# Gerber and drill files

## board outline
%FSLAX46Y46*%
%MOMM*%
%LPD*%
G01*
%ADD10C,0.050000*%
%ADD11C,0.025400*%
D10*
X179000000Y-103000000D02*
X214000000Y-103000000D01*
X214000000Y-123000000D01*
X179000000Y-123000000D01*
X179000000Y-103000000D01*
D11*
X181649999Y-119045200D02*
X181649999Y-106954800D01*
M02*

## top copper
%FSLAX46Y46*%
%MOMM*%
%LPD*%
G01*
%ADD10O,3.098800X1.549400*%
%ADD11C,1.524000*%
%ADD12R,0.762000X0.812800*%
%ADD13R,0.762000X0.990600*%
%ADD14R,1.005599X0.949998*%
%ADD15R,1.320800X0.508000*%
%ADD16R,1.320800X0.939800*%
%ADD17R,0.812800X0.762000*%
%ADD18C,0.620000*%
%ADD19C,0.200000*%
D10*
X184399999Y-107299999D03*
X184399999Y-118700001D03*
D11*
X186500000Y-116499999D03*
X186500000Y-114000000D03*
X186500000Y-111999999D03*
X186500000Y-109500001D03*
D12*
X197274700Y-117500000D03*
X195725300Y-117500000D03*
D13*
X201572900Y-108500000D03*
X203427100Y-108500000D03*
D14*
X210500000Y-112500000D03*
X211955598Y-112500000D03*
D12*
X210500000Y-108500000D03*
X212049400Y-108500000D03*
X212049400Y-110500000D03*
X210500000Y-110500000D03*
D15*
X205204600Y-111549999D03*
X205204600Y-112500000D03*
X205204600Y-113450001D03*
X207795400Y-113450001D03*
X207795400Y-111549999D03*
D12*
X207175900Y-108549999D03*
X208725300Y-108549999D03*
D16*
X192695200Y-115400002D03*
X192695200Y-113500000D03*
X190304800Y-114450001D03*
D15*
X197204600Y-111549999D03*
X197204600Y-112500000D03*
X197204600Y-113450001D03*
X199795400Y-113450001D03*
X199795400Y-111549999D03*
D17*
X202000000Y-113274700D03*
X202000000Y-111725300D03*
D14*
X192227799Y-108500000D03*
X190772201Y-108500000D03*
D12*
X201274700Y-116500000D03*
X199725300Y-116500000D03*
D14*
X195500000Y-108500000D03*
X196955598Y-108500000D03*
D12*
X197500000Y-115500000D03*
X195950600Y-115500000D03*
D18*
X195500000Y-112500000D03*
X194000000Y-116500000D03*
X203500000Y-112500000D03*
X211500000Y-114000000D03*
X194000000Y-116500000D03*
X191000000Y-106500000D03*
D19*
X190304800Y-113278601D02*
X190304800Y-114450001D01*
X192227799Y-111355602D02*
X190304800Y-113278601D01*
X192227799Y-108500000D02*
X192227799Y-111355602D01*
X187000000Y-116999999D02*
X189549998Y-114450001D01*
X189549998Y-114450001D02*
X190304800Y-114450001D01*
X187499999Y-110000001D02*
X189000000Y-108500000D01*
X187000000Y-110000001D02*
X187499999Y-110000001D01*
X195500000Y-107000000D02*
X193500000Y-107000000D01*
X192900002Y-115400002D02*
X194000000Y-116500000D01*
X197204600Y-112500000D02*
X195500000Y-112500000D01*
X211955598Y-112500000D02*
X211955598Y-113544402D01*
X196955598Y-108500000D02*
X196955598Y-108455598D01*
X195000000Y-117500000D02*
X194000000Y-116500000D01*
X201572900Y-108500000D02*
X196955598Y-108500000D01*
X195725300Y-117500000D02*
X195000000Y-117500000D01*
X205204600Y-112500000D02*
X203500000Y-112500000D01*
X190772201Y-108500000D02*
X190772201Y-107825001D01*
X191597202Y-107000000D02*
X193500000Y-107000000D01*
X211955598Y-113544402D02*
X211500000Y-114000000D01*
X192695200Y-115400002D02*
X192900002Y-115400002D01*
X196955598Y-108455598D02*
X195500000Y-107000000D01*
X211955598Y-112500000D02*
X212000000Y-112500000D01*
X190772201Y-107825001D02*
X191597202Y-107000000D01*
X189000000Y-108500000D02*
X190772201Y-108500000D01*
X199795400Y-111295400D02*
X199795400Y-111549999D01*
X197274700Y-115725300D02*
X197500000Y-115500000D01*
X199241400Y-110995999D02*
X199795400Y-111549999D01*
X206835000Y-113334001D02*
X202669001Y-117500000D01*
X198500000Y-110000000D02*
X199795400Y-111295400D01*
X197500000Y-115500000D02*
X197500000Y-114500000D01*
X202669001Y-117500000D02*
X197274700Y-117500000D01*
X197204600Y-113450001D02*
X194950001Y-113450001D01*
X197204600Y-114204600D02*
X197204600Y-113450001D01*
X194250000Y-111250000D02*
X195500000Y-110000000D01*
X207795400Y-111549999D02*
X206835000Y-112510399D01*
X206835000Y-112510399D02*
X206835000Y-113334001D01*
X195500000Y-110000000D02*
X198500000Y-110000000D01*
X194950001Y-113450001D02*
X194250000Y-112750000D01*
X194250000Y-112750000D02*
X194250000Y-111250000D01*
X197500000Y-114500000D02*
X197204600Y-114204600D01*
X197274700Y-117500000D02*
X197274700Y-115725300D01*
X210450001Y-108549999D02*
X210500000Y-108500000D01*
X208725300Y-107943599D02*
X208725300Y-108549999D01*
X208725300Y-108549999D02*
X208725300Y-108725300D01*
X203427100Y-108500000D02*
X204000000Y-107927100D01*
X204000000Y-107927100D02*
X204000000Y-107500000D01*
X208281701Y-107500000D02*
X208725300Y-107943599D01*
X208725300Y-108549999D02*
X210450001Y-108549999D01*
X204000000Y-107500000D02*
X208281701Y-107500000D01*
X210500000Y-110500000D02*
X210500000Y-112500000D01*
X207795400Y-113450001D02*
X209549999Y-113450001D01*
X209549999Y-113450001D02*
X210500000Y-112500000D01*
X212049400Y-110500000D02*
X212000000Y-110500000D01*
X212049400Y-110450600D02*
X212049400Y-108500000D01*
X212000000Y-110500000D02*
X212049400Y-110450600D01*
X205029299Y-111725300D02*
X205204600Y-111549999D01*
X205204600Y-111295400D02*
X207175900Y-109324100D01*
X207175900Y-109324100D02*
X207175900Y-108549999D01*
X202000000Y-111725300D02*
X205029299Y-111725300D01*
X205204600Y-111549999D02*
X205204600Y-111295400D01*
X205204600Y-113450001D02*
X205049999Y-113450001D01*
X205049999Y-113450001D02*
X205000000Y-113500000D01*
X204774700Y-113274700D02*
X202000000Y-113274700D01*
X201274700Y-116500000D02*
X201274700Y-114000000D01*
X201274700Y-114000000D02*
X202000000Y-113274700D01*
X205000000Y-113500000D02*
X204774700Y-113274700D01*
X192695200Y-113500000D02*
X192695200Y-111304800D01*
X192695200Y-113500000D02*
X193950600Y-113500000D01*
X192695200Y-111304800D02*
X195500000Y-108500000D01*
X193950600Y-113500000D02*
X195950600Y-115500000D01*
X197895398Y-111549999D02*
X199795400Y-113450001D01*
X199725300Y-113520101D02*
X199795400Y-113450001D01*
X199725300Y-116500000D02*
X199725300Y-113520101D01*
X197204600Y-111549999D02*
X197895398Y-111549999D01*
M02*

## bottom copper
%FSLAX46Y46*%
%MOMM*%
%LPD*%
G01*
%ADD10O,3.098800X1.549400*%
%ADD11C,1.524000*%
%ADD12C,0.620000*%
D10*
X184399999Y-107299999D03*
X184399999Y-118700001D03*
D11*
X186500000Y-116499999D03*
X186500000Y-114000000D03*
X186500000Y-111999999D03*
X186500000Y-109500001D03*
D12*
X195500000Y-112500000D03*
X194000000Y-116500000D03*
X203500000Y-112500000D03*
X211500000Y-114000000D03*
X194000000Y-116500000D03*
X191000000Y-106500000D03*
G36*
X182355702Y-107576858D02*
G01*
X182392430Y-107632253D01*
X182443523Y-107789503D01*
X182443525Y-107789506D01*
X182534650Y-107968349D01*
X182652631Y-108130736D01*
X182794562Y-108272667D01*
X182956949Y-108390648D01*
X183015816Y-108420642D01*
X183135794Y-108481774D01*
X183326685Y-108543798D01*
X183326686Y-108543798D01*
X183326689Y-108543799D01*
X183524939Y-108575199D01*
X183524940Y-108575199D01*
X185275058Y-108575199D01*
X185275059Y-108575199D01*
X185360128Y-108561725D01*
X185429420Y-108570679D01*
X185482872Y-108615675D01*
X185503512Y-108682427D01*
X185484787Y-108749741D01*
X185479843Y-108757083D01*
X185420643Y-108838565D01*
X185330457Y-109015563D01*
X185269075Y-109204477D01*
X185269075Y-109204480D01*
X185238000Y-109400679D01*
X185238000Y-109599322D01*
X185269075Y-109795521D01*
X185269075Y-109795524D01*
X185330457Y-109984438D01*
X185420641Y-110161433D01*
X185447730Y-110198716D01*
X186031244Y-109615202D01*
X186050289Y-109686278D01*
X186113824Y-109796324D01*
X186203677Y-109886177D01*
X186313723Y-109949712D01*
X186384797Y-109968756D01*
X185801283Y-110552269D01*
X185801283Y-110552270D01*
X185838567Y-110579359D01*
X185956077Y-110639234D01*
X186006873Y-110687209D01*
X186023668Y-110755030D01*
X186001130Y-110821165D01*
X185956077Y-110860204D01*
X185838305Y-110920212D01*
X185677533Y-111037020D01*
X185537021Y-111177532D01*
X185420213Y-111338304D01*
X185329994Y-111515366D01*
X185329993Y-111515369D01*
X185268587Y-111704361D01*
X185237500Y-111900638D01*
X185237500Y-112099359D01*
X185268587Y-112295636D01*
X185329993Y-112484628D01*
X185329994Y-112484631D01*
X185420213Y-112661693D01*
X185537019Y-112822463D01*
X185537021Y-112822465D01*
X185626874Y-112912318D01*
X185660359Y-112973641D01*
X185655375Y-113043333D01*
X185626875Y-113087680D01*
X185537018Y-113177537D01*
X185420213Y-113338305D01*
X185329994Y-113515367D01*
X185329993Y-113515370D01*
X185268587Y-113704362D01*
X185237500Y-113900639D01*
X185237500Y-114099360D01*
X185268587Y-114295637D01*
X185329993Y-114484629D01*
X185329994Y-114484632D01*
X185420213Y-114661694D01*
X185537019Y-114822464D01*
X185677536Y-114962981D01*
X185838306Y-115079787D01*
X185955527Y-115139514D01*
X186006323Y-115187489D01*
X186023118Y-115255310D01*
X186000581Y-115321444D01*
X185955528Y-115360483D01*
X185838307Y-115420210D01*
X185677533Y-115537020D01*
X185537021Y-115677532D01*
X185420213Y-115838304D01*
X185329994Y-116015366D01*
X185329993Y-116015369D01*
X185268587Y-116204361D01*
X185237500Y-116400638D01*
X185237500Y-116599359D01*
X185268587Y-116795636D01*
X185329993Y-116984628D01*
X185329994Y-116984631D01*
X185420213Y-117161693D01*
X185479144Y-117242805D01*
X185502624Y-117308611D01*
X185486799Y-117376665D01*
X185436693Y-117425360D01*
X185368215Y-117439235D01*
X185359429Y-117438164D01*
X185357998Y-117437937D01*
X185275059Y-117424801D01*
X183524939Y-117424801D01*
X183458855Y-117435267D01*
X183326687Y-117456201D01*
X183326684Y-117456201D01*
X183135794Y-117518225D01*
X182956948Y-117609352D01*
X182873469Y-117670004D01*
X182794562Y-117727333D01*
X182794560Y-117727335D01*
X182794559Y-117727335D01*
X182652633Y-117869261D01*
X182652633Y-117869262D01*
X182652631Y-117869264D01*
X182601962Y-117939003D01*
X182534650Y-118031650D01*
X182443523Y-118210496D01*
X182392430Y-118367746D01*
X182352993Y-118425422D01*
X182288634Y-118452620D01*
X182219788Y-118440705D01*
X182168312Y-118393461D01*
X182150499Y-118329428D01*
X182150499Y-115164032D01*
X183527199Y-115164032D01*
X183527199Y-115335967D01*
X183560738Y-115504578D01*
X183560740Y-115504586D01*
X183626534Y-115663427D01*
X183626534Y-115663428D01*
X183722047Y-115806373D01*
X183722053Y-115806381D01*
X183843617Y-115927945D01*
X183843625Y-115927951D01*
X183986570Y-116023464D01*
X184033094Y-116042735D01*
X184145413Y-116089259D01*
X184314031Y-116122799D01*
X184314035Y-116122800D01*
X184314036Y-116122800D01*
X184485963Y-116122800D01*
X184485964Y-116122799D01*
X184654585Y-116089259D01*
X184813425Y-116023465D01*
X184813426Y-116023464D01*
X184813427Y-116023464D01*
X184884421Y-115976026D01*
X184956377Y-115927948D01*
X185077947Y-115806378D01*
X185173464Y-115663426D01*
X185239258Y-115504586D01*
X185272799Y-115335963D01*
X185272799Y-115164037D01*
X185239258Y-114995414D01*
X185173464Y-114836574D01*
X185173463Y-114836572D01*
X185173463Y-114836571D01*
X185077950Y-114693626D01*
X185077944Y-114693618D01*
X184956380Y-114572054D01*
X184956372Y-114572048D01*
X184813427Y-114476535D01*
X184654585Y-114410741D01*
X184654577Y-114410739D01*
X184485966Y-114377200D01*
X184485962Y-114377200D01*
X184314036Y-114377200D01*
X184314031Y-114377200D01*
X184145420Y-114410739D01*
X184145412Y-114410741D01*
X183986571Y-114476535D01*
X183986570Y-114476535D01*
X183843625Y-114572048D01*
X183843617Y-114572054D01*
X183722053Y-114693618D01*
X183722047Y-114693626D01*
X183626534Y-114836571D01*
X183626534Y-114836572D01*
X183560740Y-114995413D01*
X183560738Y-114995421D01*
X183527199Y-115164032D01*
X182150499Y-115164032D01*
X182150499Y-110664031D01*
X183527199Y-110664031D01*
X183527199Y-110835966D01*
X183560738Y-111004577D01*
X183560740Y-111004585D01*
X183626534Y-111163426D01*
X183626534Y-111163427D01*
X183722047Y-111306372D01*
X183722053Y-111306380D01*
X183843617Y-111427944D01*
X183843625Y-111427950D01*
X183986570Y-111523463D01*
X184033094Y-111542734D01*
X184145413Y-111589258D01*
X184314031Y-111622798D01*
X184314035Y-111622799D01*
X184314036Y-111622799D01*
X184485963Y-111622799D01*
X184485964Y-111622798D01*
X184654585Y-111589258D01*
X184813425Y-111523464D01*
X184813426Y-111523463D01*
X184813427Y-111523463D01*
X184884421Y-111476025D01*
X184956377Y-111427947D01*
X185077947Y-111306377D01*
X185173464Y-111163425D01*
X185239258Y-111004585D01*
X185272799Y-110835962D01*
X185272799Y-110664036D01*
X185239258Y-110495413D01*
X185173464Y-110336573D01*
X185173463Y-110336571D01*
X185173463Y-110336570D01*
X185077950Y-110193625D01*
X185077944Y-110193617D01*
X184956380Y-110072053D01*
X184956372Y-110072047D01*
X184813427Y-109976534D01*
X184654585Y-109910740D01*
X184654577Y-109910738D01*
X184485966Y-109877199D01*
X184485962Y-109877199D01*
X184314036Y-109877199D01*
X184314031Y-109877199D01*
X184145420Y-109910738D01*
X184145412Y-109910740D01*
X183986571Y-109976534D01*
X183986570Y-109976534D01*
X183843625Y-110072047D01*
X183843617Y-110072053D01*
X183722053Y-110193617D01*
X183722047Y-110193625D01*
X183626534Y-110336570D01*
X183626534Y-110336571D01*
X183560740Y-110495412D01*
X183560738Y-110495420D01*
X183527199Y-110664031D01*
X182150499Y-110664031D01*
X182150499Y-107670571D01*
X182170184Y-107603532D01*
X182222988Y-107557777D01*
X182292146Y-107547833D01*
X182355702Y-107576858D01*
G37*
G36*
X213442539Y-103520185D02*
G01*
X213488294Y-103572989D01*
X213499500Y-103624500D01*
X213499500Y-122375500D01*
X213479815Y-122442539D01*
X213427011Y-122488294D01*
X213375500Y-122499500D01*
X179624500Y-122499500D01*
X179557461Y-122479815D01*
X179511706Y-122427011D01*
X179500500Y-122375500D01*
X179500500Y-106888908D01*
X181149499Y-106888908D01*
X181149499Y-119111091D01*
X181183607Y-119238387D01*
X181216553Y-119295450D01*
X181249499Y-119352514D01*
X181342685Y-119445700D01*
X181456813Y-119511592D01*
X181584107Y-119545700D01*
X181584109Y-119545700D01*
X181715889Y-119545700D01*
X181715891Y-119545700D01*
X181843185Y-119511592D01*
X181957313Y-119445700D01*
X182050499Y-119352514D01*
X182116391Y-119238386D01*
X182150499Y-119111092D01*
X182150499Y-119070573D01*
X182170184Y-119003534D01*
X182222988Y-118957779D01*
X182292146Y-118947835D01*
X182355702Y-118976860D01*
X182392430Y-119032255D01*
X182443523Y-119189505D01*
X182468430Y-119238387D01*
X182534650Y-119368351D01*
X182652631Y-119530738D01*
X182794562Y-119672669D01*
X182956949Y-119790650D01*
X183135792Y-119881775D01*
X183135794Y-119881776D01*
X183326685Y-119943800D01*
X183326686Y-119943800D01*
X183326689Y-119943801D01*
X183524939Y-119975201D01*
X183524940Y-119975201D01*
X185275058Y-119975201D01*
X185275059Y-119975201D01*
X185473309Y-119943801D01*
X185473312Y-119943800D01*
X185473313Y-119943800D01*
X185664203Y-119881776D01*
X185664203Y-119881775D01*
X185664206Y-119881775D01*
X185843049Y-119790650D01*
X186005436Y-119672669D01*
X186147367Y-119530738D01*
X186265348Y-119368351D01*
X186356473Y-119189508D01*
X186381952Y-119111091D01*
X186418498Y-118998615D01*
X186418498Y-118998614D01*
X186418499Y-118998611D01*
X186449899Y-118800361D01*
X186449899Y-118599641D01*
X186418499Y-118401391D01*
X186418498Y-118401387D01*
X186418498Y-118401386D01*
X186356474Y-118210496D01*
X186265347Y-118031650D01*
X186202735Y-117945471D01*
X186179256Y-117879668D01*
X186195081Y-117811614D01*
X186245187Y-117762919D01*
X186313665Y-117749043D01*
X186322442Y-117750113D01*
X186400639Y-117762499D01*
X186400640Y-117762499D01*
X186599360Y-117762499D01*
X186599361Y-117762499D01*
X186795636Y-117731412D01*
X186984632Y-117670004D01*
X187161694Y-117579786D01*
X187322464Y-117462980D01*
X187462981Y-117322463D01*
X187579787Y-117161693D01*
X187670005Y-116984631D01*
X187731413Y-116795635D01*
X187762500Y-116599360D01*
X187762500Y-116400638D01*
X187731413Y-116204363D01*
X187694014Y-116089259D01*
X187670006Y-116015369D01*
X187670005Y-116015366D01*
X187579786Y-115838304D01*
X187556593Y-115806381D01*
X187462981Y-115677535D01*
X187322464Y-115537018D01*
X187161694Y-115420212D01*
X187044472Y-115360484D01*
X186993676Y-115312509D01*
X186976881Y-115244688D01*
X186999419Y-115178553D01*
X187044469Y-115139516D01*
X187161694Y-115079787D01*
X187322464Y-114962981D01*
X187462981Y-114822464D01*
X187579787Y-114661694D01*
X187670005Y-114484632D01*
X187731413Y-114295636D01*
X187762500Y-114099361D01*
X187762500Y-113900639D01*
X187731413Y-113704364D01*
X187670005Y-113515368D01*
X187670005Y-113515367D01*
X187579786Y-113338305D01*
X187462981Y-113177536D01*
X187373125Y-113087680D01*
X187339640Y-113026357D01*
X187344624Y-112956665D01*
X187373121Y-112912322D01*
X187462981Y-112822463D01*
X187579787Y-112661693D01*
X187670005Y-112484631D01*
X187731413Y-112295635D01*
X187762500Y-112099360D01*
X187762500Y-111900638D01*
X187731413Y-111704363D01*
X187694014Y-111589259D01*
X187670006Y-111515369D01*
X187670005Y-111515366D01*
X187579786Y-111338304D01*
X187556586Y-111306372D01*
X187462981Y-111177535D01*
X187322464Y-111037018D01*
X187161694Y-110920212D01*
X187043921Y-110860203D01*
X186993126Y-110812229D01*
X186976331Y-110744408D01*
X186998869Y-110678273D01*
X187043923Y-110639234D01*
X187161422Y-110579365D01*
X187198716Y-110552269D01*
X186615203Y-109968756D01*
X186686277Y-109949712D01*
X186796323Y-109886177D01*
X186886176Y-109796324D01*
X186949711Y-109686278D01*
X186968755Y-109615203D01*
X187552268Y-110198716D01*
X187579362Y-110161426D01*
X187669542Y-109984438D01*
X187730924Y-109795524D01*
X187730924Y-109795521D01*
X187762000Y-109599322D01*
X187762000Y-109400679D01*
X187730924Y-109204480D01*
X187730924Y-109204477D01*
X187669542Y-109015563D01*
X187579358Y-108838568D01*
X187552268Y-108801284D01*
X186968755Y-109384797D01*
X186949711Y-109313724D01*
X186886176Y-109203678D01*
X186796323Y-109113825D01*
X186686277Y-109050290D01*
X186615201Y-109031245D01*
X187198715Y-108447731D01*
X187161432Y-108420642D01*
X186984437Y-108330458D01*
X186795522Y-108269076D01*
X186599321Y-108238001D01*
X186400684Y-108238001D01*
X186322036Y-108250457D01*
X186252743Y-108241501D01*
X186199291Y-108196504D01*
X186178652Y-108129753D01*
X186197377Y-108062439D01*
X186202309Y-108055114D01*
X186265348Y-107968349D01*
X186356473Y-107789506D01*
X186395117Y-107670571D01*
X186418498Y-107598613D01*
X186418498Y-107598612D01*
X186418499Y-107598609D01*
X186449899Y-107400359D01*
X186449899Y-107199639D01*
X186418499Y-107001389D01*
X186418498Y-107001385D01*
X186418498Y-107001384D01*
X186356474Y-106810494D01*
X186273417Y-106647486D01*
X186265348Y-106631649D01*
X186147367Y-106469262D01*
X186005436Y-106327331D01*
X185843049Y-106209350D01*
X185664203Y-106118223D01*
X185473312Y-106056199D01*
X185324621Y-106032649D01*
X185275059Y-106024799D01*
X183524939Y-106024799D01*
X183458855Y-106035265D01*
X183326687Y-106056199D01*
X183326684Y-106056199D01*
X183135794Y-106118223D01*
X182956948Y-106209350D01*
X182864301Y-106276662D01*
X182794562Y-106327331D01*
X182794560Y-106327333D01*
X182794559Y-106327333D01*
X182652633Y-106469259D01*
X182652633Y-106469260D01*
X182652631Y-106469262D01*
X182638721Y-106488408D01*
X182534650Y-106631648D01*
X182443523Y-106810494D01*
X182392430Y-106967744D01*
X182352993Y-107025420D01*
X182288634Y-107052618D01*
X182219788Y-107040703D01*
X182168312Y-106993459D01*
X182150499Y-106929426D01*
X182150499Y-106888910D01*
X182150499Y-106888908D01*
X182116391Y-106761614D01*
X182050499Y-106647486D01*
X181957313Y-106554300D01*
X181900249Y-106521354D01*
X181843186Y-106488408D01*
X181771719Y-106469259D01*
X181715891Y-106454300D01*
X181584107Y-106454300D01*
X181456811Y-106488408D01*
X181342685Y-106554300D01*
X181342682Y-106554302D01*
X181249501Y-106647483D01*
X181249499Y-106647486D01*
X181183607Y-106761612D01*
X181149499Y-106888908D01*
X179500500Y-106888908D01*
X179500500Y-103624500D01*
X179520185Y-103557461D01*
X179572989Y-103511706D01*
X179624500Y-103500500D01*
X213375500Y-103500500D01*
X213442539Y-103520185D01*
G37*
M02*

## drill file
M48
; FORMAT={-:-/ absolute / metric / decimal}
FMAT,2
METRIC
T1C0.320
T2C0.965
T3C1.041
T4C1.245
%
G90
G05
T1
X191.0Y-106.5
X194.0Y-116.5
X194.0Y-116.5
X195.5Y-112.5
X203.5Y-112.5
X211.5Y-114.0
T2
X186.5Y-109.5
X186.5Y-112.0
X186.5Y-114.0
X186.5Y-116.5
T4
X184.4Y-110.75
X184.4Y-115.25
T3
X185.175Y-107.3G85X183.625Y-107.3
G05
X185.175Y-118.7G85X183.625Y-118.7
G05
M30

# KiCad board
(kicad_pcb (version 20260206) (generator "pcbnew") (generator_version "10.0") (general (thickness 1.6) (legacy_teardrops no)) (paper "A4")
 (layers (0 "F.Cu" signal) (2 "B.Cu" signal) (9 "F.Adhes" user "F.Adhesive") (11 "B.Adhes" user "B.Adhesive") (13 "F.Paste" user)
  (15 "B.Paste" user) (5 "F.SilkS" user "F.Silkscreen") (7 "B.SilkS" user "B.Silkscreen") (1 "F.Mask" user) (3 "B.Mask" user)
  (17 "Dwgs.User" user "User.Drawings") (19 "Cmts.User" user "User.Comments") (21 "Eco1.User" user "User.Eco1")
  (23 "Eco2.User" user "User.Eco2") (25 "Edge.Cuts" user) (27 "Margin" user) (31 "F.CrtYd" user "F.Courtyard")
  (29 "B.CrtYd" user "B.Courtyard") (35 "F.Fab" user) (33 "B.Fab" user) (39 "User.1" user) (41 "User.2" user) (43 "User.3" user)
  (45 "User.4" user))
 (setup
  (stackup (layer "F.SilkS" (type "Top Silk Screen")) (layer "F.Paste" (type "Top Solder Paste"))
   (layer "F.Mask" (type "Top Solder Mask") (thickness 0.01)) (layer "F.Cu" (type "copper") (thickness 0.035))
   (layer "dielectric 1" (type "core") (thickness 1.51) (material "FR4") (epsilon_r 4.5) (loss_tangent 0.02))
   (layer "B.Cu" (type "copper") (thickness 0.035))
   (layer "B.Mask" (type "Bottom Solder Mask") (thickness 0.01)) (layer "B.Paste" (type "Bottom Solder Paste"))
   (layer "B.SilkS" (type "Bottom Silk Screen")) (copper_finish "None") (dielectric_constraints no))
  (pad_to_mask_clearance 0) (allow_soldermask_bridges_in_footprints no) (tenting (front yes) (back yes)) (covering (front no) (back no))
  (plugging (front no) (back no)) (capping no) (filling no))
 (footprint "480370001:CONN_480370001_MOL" (layer "F.Cu") (at 186.5 116.499999 -90)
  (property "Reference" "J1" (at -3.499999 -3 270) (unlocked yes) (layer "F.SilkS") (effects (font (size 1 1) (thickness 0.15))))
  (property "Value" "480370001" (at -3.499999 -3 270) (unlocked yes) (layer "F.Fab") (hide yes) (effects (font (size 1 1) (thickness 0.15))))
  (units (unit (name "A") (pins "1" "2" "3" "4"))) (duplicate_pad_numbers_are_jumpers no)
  (fp_line (start 2.545201 4.850001) (end -9.545199 4.850001) (stroke (width 0.0254) (type solid)) (layer "Edge.Cuts"))
  (pad "" np_thru_hole oval (at -9.2 2.100001 270) (size 1.5494 3.0988) (drill oval 1.0414 2.5908) (layers "*.Cu" "*.Mask"))
  (pad "" np_thru_hole circle (at -5.75 2.100001 270) (size 1.2446 1.2446) (drill 1.2446) (layers))
  (pad "" np_thru_hole circle (at -1.249999 2.100001 270) (size 1.2446 1.2446) (drill 1.2446) (layers))
  (pad "" np_thru_hole oval (at 2.200002 2.100001 270) (size 1.5494 3.0988) (drill oval 1.0414 2.5908) (layers "*.Cu" "*.Mask"))
  (pad "1" thru_hole circle (at 0 0 270) (size 1.524 1.524) (drill 0.9652) (layers "*.Cu" "*.Mask") (remove_unused_layers no)
   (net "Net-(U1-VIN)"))
  (pad "2" thru_hole circle (at -2.499999 0 270) (size 1.524 1.524) (drill 0.9652) (layers "*.Cu" "*.Mask") (remove_unused_layers no)
   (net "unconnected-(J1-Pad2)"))
  (pad "3" thru_hole circle (at -4.5 0 270) (size 1.524 1.524) (drill 0.9652) (layers "*.Cu" "*.Mask") (remove_unused_layers no)
   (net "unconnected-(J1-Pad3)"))
  (pad "4" thru_hole circle (at -6.999998 0 270) (size 1.524 1.524) (drill 0.9652) (layers "*.Cu" "*.Mask") (remove_unused_layers no)
   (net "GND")))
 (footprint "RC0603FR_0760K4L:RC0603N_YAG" (layer "F.Cu") (at 196.5 117.5 180)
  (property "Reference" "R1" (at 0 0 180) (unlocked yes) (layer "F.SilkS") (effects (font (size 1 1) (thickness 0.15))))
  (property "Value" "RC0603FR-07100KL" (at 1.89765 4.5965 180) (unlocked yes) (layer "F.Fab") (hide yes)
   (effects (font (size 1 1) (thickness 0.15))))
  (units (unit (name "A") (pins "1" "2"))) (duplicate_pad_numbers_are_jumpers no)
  (pad "1" smd rect (at -0.7747 0 180) (size 0.762 0.8128) (layers "F.Cu" "F.Mask" "F.Paste") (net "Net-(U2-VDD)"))
  (pad "2" smd rect (at 0.7747 0 180) (size 0.762 0.8128) (layers "F.Cu" "F.Mask" "F.Paste") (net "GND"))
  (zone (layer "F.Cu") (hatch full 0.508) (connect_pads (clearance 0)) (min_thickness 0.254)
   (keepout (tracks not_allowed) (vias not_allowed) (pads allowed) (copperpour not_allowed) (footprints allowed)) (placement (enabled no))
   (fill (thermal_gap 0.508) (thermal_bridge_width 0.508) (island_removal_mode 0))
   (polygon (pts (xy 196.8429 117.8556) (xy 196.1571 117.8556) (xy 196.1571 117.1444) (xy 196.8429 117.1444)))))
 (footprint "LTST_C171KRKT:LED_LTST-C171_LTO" (layer "F.Cu") (at 202.5 108.5)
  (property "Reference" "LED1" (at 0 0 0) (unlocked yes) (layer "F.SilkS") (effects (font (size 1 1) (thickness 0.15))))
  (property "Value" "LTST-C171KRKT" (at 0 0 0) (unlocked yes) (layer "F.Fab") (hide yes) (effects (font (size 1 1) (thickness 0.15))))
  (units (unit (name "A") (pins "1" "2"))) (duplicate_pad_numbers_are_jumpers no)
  (pad "1" smd rect (at -0.9271 0) (size 0.762 0.9906) (layers "F.Cu" "F.Mask" "F.Paste") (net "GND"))
  (pad "2" smd rect (at 0.9271 0) (size 0.762 0.9906) (layers "F.Cu" "F.Mask" "F.Paste") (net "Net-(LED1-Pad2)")))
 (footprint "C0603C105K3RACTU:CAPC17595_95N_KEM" (layer "F.Cu") (at 211.227799 112.5)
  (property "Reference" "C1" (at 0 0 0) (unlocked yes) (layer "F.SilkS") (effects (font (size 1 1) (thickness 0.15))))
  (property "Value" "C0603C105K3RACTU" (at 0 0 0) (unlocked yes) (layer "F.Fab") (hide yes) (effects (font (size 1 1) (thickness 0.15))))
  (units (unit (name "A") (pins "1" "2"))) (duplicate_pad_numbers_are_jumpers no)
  (pad "1" smd rect (at -0.727799 0) (size 1.005599 0.949998) (layers "F.Cu" "F.Mask" "F.Paste") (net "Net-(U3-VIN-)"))
  (pad "2" smd rect (at 0.727799 0) (size 1.005599 0.949998) (layers "F.Cu" "F.Mask" "F.Paste") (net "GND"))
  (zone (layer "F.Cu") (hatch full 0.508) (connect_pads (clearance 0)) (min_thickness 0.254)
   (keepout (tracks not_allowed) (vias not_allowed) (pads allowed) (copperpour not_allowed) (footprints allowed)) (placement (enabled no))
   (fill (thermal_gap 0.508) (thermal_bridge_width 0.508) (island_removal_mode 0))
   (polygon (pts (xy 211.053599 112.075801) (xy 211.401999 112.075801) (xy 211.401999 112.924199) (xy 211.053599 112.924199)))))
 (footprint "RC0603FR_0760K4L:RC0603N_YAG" (layer "F.Cu") (at 211.2747 108.5)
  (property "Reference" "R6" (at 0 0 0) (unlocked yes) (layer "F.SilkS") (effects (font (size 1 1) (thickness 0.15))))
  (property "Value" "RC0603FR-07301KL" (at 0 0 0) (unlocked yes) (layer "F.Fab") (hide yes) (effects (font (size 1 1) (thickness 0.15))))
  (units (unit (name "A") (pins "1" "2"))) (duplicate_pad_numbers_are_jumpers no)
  (pad "1" smd rect (at -0.7747 0) (size 0.762 0.8128) (layers "F.Cu" "F.Mask" "F.Paste") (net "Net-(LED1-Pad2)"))
  (pad "2" smd rect (at 0.7747 0) (size 0.762 0.8128) (layers "F.Cu" "F.Mask" "F.Paste") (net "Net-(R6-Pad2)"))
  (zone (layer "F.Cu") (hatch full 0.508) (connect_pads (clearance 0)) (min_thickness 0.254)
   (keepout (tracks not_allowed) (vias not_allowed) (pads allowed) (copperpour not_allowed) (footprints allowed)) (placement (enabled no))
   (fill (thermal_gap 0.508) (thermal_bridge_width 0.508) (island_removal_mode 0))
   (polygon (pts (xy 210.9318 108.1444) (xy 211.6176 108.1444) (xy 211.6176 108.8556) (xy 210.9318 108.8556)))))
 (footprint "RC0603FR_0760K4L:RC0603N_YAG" (layer "F.Cu") (at 211.2747 110.5 180)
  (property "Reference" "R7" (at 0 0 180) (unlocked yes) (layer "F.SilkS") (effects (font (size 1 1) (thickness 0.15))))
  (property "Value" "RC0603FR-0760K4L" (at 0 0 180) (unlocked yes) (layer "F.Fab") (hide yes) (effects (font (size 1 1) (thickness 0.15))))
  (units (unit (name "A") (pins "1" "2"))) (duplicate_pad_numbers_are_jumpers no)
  (pad "1" smd rect (at -0.7747 0 180) (size 0.762 0.8128) (layers "F.Cu" "F.Mask" "F.Paste") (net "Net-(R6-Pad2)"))
  (pad "2" smd rect (at 0.7747 0 180) (size 0.762 0.8128) (layers "F.Cu" "F.Mask" "F.Paste") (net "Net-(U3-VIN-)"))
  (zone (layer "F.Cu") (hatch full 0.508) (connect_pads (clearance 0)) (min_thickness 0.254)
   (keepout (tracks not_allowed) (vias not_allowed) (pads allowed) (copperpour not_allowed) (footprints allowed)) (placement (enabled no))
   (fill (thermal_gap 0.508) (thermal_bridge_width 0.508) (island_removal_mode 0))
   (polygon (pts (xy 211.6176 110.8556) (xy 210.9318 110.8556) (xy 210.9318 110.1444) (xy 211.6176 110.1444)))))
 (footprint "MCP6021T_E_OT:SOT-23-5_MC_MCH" (layer "F.Cu") (at 206.5 112.5)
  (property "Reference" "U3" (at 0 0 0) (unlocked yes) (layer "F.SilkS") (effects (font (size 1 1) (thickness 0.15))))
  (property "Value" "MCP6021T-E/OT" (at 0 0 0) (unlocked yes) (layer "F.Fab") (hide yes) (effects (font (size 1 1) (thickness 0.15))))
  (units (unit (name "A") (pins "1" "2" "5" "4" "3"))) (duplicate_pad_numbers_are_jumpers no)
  (pad "1" smd rect (at -1.2954 -0.950001) (size 1.3208 0.508) (layers "F.Cu" "F.Mask" "F.Paste") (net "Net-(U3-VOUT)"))
  (pad "2" smd rect (at -1.2954 0) (size 1.3208 0.508) (layers "F.Cu" "F.Mask" "F.Paste") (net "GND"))
  (pad "3" smd rect (at -1.2954 0.950001) (size 1.3208 0.508) (layers "F.Cu" "F.Mask" "F.Paste") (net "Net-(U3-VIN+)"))
  (pad "4" smd rect (at 1.2954 0.950001) (size 1.3208 0.508) (layers "F.Cu" "F.Mask" "F.Paste") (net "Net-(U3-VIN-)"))
  (pad "5" smd rect (at 1.2954 -0.950001) (size 1.3208 0.508) (layers "F.Cu" "F.Mask" "F.Paste") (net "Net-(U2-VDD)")))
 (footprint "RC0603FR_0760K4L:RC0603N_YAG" (layer "F.Cu") (at 207.9506 108.549999)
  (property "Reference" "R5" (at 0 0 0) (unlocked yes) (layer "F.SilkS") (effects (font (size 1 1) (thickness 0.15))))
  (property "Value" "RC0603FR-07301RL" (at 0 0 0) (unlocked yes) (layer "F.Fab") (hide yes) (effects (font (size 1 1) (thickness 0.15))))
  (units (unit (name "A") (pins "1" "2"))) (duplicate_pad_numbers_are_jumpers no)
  (pad "1" smd rect (at -0.7747 0) (size 0.762 0.8128) (layers "F.Cu" "F.Mask" "F.Paste") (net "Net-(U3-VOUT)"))
  (pad "2" smd rect (at 0.7747 0) (size 0.762 0.8128) (layers "F.Cu" "F.Mask" "F.Paste") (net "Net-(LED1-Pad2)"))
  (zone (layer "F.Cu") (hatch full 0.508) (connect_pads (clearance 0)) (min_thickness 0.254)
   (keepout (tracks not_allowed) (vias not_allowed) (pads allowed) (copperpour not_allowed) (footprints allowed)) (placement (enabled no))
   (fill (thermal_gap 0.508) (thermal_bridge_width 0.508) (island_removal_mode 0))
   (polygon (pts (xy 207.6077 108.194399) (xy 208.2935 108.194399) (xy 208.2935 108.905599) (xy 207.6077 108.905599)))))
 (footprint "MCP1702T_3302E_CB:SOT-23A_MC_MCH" (layer "F.Cu") (at 191.5 114.450001 90)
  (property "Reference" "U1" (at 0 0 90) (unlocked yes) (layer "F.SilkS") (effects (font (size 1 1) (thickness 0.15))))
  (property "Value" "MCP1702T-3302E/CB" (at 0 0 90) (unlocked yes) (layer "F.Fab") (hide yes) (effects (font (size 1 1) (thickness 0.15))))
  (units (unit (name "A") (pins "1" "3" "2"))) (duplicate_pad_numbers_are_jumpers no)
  (pad "1" smd rect (at -0.950001 1.1952 90) (size 0.9398 1.3208) (layers "F.Cu" "F.Mask" "F.Paste") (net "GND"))
  (pad "2" smd rect (at 0.950001 1.1952 90) (size 0.9398 1.3208) (layers "F.Cu" "F.Mask" "F.Paste") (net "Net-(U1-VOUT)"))
  (pad "3" smd rect (at 0 -1.1952 90) (size 0.9398 1.3208) (layers "F.Cu" "F.Mask" "F.Paste") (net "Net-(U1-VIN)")))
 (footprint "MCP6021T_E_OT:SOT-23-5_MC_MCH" (layer "F.Cu") (at 198.5 112.5)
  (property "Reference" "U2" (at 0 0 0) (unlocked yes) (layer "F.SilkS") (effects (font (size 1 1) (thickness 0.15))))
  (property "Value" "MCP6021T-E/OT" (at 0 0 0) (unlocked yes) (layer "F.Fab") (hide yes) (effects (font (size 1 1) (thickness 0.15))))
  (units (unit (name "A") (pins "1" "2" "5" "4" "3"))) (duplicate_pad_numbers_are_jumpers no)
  (pad "1" smd rect (at -1.2954 -0.950001) (size 1.3208 0.508) (layers "F.Cu" "F.Mask" "F.Paste") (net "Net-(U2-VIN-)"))
  (pad "2" smd rect (at -1.2954 0) (size 1.3208 0.508) (layers "F.Cu" "F.Mask" "F.Paste") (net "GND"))
  (pad "3" smd rect (at -1.2954 0.950001) (size 1.3208 0.508) (layers "F.Cu" "F.Mask" "F.Paste") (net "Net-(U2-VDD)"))
  (pad "4" smd rect (at 1.2954 0.950001) (size 1.3208 0.508) (layers "F.Cu" "F.Mask" "F.Paste") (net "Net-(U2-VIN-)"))
  (pad "5" smd rect (at 1.2954 -0.950001) (size 1.3208 0.508) (layers "F.Cu" "F.Mask" "F.Paste") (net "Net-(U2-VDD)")))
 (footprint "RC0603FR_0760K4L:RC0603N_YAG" (layer "F.Cu") (at 202 112.5 90)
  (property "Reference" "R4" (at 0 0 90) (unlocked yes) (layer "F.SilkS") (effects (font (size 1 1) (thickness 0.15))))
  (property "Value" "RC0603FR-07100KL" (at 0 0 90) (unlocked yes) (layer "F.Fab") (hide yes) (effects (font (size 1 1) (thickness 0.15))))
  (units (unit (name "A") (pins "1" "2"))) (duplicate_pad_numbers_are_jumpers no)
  (pad "1" smd rect (at -0.7747 0 90) (size 0.762 0.8128) (layers "F.Cu" "F.Mask" "F.Paste") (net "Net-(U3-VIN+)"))
  (pad "2" smd rect (at 0.7747 0 90) (size 0.762 0.8128) (layers "F.Cu" "F.Mask" "F.Paste") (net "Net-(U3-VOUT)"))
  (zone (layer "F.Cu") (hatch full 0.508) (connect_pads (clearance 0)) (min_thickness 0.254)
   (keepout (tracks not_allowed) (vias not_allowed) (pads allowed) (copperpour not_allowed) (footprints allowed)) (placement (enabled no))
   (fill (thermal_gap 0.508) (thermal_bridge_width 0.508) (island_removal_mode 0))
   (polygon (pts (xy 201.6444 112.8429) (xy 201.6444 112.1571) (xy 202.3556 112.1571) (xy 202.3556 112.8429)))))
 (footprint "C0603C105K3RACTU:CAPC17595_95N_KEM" (layer "F.Cu") (at 191.5 108.5 180)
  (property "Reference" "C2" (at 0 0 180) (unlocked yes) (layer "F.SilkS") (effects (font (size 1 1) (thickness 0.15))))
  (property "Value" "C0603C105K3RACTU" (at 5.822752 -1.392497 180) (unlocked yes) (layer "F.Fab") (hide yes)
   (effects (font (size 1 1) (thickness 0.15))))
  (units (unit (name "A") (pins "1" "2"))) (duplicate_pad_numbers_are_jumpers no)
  (pad "1" smd rect (at -0.727799 0 180) (size 1.005599 0.949998) (layers "F.Cu" "F.Mask" "F.Paste") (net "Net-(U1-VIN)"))
  (pad "2" smd rect (at 0.727799 0 180) (size 1.005599 0.949998) (layers "F.Cu" "F.Mask" "F.Paste") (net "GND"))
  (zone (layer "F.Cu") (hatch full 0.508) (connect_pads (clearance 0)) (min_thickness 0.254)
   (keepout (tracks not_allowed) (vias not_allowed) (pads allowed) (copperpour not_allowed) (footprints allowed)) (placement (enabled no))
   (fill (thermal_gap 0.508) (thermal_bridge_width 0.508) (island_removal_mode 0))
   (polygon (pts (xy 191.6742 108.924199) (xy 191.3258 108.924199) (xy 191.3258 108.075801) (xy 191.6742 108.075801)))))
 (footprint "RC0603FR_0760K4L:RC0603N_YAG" (layer "F.Cu") (at 200.5 116.5 180)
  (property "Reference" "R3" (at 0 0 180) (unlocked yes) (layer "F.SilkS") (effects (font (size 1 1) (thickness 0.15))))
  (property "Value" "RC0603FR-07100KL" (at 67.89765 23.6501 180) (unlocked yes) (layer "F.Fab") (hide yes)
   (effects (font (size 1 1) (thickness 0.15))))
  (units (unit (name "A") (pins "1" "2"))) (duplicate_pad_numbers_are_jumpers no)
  (pad "1" smd rect (at -0.7747 0 180) (size 0.762 0.8128) (layers "F.Cu" "F.Mask" "F.Paste") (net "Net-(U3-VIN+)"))
  (pad "2" smd rect (at 0.7747 0 180) (size 0.762 0.8128) (layers "F.Cu" "F.Mask" "F.Paste") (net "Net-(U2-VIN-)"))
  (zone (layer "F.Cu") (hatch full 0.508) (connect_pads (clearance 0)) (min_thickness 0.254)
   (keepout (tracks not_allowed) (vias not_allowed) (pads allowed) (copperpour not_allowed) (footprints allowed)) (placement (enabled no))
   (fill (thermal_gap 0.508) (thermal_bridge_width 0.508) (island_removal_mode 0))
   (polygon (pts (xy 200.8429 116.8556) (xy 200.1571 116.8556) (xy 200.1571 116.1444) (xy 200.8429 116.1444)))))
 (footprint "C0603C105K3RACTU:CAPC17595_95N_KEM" (layer "F.Cu") (at 196.227799 108.5)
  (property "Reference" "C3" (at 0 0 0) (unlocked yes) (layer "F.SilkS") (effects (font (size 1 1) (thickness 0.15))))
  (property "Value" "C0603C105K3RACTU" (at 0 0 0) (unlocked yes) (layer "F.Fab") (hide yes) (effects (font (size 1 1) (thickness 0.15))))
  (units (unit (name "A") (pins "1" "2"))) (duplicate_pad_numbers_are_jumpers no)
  (pad "1" smd rect (at -0.727799 0) (size 1.005599 0.949998) (layers "F.Cu" "F.Mask" "F.Paste") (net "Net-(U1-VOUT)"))
  (pad "2" smd rect (at 0.727799 0) (size 1.005599 0.949998) (layers "F.Cu" "F.Mask" "F.Paste") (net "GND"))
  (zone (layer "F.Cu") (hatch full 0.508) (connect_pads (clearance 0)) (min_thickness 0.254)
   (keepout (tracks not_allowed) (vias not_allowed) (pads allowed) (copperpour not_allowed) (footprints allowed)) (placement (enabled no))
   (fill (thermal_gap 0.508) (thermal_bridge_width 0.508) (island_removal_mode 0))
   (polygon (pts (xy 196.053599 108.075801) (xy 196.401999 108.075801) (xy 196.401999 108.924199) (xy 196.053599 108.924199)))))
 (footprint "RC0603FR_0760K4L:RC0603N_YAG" (layer "F.Cu") (at 196.7253 115.5 180)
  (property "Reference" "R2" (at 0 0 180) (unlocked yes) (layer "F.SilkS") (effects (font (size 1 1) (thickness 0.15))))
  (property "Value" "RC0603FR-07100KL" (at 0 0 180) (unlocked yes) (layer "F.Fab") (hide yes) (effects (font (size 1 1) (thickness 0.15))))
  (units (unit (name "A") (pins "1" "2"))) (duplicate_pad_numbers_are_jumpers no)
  (pad "1" smd rect (at -0.7747 0 180) (size 0.762 0.8128) (layers "F.Cu" "F.Mask" "F.Paste") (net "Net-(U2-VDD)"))
  (pad "2" smd rect (at 0.7747 0 180) (size 0.762 0.8128) (layers "F.Cu" "F.Mask" "F.Paste") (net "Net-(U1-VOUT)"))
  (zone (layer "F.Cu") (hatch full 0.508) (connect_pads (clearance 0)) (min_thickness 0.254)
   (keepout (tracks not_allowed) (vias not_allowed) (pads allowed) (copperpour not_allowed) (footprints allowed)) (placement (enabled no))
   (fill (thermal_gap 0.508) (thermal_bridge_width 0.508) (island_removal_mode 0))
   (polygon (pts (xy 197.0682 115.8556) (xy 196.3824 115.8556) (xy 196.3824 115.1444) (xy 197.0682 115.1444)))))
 (gr_rect (start 179 103) (end 214 123) (stroke (width 0.05) (type default)) (fill no) (layer "Edge.Cuts"))
 (segment (start 190.3048 113.278601) (end 190.3048 114.450001) (width 0.2) (layer "F.Cu") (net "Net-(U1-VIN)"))
 (segment (start 192.227799 111.355602) (end 190.3048 113.278601) (width 0.2) (layer "F.Cu") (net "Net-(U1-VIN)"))
 (segment (start 192.227799 108.5) (end 192.227799 111.355602) (width 0.2) (layer "F.Cu") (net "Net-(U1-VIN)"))
 (segment (start 187 116.999999) (end 189.549998 114.450001) (width 0.2) (layer "F.Cu") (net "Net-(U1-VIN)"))
 (segment (start 189.549998 114.450001) (end 190.3048 114.450001) (width 0.2) (layer "F.Cu") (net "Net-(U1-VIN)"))
 (segment (start 187.499999 110.000001) (end 189 108.5) (width 0.2) (layer "F.Cu") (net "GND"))
 (segment (start 187 110.000001) (end 187.499999 110.000001) (width 0.2) (layer "F.Cu") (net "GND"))
 (segment (start 195.5 107) (end 193.5 107) (width 0.2) (layer "F.Cu") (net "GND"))
 (segment (start 192.900002 115.400002) (end 194 116.5) (width 0.2) (layer "F.Cu") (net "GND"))
 (segment (start 197.2046 112.5) (end 195.5 112.5) (width 0.2) (layer "F.Cu") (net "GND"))
 (segment (start 211.955598 112.5) (end 211.955598 113.544402) (width 0.2) (layer "F.Cu") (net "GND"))
 (segment (start 196.955598 108.5) (end 196.955598 108.455598) (width 0.2) (layer "F.Cu") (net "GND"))
 (segment (start 195 117.5) (end 194 116.5) (width 0.2) (layer "F.Cu") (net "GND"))
 (segment (start 201.5729 108.5) (end 196.955598 108.5) (width 0.2) (layer "F.Cu") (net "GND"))
 (segment (start 195.7253 117.5) (end 195 117.5) (width 0.2) (layer "F.Cu") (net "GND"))
 (segment (start 205.2046 112.5) (end 203.5 112.5) (width 0.2) (layer "F.Cu") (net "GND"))
 (segment (start 190.772201 108.5) (end 190.772201 107.825001) (width 0.2) (layer "F.Cu") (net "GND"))
 (segment (start 191.597202 107) (end 193.5 107) (width 0.2) (layer "F.Cu") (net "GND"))
 (segment (start 211.955598 113.544402) (end 211.5 114) (width 0.2) (layer "F.Cu") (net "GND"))
 (segment (start 192.6952 115.400002) (end 192.900002 115.400002) (width 0.2) (layer "F.Cu") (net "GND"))
 (segment (start 196.955598 108.455598) (end 195.5 107) (width 0.2) (layer "F.Cu") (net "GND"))
 (segment (start 211.955598 112.5) (end 212 112.5) (width 0.2) (layer "F.Cu") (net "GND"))
 (segment (start 190.772201 107.825001) (end 191.597202 107) (width 0.2) (layer "F.Cu") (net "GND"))
 (segment (start 189 108.5) (end 190.772201 108.5) (width 0.2) (layer "F.Cu") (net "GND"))
 (via (at 195.5 112.5) (size 0.62) (drill 0.32) (layers "F.Cu" "B.Cu") (free yes) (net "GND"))
 (via (at 194 116.5) (size 0.62) (drill 0.32) (layers "F.Cu" "B.Cu") (free yes) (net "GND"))
 (via (at 203.5 112.5) (size 0.62) (drill 0.32) (layers "F.Cu" "B.Cu") (free yes) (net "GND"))
 (via (at 211.5 114) (size 0.62) (drill 0.32) (layers "F.Cu" "B.Cu") (free yes) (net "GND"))
 (via (at 194 116.5) (size 0.62) (drill 0.32) (layers "F.Cu" "B.Cu") (free yes) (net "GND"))
 (via (at 191 106.5) (size 0.62) (drill 0.32) (layers "F.Cu" "B.Cu") (free yes) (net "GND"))
 (segment (start 199.7954 111.2954) (end 199.7954 111.549999) (width 0.2) (layer "F.Cu") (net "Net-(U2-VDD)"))
 (segment (start 197.2747 115.7253) (end 197.5 115.5) (width 0.2) (layer "F.Cu") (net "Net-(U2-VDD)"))
 (segment (start 199.2414 110.995999) (end 199.7954 111.549999) (width 0.2) (layer "F.Cu") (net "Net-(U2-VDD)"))
 (segment (start 206.835 113.334001) (end 202.669001 117.5) (width 0.2) (layer "F.Cu") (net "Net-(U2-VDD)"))
 (segment (start 198.5 110) (end 199.7954 111.2954) (width 0.2) (layer "F.Cu") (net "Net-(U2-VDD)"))
 (segment (start 197.5 115.5) (end 197.5 114.5) (width 0.2) (layer "F.Cu") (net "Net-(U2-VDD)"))
 (segment (start 202.669001 117.5) (end 197.2747 117.5) (width 0.2) (layer "F.Cu") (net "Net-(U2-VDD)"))
 (segment (start 197.2046 113.450001) (end 194.950001 113.450001) (width 0.2) (layer "F.Cu") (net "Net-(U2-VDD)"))
 (segment (start 197.2046 114.2046) (end 197.2046 113.450001) (width 0.2) (layer "F.Cu") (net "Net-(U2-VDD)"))
 (segment (start 194.25 111.25) (end 195.5 110) (width 0.2) (layer "F.Cu") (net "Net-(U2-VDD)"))
 (segment (start 207.7954 111.549999) (end 206.835 112.510399) (width 0.2) (layer "F.Cu") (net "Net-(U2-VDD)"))
 (segment (start 206.835 112.510399) (end 206.835 113.334001) (width 0.2) (layer "F.Cu") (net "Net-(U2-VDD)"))
 (segment (start 195.5 110) (end 198.5 110) (width 0.2) (layer "F.Cu") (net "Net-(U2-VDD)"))
 (segment (start 194.950001 113.450001) (end 194.25 112.75) (width 0.2) (layer "F.Cu") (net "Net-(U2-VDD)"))
 (segment (start 194.25 112.75) (end 194.25 111.25) (width 0.2) (layer "F.Cu") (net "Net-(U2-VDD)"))
 (segment (start 197.5 114.5) (end 197.2046 114.2046) (width 0.2) (layer "F.Cu") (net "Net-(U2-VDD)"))
 (segment (start 197.2747 117.5) (end 197.2747 115.7253) (width 0.2) (layer "F.Cu") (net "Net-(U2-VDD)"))
 (segment (start 210.450001 108.549999) (end 210.5 108.5) (width 0.2) (layer "F.Cu") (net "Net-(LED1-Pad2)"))
 (segment (start 208.7253 107.943599) (end 208.7253 108.549999) (width 0.2) (layer "F.Cu") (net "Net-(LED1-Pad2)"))
 (segment (start 208.7253 108.549999) (end 208.7253 108.7253) (width 0.2) (layer "F.Cu") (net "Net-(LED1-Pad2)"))
 (segment (start 203.4271 108.5) (end 204 107.9271) (width 0.2) (layer "F.Cu") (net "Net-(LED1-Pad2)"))
 (segment (start 204 107.9271) (end 204 107.5) (width 0.2) (layer "F.Cu") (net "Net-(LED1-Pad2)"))
 (segment (start 208.281701 107.5) (end 208.7253 107.943599) (width 0.2) (layer "F.Cu") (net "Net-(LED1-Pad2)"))
 (segment (start 208.7253 108.549999) (end 210.450001 108.549999) (width 0.2) (layer "F.Cu") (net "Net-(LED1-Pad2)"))
 (segment (start 204 107.5) (end 208.281701 107.5) (width 0.2) (layer "F.Cu") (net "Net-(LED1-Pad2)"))
 (segment (start 210.5 110.5) (end 210.5 112.5) (width 0.2) (layer "F.Cu") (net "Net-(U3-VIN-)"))
 (segment (start 207.7954 113.450001) (end 209.549999 113.450001) (width 0.2) (layer "F.Cu") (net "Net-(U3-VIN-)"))
 (segment (start 209.549999 113.450001) (end 210.5 112.5) (width 0.2) (layer "F.Cu") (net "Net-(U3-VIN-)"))
 (segment (start 212.0494 110.5) (end 212 110.5) (width 0.2) (layer "F.Cu") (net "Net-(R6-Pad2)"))
 (segment (start 212.0494 110.4506) (end 212.0494 108.5) (width 0.2) (layer "F.Cu") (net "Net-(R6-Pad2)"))
 (segment (start 212 110.5) (end 212.0494 110.4506) (width 0.2) (layer "F.Cu") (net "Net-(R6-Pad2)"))
 (segment (start 205.029299 111.7253) (end 205.2046 111.549999) (width 0.2) (layer "F.Cu") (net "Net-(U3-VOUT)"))
 (segment (start 205.2046 111.2954) (end 207.1759 109.3241) (width 0.2) (layer "F.Cu") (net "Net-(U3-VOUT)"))
 (segment (start 207.1759 109.3241) (end 207.1759 108.549999) (width 0.2) (layer "F.Cu") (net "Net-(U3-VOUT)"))
 (segment (start 202 111.7253) (end 205.029299 111.7253) (width 0.2) (layer "F.Cu") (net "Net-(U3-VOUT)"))
 (segment (start 205.2046 111.549999) (end 205.2046 111.2954) (width 0.2) (layer "F.Cu") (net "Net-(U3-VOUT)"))
 (segment (start 205.2046 113.450001) (end 205.049999 113.450001) (width 0.2) (layer "F.Cu") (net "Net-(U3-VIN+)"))
 (segment (start 205.049999 113.450001) (end 205 113.5) (width 0.2) (layer "F.Cu") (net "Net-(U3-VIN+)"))
 (segment (start 204.7747 113.2747) (end 202 113.2747) (width 0.2) (layer "F.Cu") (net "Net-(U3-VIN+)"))
 (segment (start 201.2747 116.5) (end 201.2747 114) (width 0.2) (layer "F.Cu") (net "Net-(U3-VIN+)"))
 (segment (start 201.2747 114) (end 202 113.2747) (width 0.2) (layer "F.Cu") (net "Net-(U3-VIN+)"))
 (segment (start 205 113.5) (end 204.7747 113.2747) (width 0.2) (layer "F.Cu") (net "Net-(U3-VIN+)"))
 (segment (start 192.6952 113.5) (end 192.6952 111.3048) (width 0.2) (layer "F.Cu") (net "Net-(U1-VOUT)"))
 (segment (start 192.6952 113.5) (end 193.9506 113.5) (width 0.2) (layer "F.Cu") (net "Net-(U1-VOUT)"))
 (segment (start 192.6952 111.3048) (end 195.5 108.5) (width 0.2) (layer "F.Cu") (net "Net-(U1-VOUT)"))
 (segment (start 193.9506 113.5) (end 195.9506 115.5) (width 0.2) (layer "F.Cu") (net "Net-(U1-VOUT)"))
 (segment (start 197.895398 111.549999) (end 199.7954 113.450001) (width 0.2) (layer "F.Cu") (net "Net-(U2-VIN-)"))
 (segment (start 199.7253 113.520101) (end 199.7954 113.450001) (width 0.2) (layer "F.Cu") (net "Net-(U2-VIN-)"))
 (segment (start 199.7253 116.5) (end 199.7253 113.520101) (width 0.2) (layer "F.Cu") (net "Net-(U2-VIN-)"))
 (segment (start 197.2046 111.549999) (end 197.895398 111.549999) (width 0.2) (layer "F.Cu") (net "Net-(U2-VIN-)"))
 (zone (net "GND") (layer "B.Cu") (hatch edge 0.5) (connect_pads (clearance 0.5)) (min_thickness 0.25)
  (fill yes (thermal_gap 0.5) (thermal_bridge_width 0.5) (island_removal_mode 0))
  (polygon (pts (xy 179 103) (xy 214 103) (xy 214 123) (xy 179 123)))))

